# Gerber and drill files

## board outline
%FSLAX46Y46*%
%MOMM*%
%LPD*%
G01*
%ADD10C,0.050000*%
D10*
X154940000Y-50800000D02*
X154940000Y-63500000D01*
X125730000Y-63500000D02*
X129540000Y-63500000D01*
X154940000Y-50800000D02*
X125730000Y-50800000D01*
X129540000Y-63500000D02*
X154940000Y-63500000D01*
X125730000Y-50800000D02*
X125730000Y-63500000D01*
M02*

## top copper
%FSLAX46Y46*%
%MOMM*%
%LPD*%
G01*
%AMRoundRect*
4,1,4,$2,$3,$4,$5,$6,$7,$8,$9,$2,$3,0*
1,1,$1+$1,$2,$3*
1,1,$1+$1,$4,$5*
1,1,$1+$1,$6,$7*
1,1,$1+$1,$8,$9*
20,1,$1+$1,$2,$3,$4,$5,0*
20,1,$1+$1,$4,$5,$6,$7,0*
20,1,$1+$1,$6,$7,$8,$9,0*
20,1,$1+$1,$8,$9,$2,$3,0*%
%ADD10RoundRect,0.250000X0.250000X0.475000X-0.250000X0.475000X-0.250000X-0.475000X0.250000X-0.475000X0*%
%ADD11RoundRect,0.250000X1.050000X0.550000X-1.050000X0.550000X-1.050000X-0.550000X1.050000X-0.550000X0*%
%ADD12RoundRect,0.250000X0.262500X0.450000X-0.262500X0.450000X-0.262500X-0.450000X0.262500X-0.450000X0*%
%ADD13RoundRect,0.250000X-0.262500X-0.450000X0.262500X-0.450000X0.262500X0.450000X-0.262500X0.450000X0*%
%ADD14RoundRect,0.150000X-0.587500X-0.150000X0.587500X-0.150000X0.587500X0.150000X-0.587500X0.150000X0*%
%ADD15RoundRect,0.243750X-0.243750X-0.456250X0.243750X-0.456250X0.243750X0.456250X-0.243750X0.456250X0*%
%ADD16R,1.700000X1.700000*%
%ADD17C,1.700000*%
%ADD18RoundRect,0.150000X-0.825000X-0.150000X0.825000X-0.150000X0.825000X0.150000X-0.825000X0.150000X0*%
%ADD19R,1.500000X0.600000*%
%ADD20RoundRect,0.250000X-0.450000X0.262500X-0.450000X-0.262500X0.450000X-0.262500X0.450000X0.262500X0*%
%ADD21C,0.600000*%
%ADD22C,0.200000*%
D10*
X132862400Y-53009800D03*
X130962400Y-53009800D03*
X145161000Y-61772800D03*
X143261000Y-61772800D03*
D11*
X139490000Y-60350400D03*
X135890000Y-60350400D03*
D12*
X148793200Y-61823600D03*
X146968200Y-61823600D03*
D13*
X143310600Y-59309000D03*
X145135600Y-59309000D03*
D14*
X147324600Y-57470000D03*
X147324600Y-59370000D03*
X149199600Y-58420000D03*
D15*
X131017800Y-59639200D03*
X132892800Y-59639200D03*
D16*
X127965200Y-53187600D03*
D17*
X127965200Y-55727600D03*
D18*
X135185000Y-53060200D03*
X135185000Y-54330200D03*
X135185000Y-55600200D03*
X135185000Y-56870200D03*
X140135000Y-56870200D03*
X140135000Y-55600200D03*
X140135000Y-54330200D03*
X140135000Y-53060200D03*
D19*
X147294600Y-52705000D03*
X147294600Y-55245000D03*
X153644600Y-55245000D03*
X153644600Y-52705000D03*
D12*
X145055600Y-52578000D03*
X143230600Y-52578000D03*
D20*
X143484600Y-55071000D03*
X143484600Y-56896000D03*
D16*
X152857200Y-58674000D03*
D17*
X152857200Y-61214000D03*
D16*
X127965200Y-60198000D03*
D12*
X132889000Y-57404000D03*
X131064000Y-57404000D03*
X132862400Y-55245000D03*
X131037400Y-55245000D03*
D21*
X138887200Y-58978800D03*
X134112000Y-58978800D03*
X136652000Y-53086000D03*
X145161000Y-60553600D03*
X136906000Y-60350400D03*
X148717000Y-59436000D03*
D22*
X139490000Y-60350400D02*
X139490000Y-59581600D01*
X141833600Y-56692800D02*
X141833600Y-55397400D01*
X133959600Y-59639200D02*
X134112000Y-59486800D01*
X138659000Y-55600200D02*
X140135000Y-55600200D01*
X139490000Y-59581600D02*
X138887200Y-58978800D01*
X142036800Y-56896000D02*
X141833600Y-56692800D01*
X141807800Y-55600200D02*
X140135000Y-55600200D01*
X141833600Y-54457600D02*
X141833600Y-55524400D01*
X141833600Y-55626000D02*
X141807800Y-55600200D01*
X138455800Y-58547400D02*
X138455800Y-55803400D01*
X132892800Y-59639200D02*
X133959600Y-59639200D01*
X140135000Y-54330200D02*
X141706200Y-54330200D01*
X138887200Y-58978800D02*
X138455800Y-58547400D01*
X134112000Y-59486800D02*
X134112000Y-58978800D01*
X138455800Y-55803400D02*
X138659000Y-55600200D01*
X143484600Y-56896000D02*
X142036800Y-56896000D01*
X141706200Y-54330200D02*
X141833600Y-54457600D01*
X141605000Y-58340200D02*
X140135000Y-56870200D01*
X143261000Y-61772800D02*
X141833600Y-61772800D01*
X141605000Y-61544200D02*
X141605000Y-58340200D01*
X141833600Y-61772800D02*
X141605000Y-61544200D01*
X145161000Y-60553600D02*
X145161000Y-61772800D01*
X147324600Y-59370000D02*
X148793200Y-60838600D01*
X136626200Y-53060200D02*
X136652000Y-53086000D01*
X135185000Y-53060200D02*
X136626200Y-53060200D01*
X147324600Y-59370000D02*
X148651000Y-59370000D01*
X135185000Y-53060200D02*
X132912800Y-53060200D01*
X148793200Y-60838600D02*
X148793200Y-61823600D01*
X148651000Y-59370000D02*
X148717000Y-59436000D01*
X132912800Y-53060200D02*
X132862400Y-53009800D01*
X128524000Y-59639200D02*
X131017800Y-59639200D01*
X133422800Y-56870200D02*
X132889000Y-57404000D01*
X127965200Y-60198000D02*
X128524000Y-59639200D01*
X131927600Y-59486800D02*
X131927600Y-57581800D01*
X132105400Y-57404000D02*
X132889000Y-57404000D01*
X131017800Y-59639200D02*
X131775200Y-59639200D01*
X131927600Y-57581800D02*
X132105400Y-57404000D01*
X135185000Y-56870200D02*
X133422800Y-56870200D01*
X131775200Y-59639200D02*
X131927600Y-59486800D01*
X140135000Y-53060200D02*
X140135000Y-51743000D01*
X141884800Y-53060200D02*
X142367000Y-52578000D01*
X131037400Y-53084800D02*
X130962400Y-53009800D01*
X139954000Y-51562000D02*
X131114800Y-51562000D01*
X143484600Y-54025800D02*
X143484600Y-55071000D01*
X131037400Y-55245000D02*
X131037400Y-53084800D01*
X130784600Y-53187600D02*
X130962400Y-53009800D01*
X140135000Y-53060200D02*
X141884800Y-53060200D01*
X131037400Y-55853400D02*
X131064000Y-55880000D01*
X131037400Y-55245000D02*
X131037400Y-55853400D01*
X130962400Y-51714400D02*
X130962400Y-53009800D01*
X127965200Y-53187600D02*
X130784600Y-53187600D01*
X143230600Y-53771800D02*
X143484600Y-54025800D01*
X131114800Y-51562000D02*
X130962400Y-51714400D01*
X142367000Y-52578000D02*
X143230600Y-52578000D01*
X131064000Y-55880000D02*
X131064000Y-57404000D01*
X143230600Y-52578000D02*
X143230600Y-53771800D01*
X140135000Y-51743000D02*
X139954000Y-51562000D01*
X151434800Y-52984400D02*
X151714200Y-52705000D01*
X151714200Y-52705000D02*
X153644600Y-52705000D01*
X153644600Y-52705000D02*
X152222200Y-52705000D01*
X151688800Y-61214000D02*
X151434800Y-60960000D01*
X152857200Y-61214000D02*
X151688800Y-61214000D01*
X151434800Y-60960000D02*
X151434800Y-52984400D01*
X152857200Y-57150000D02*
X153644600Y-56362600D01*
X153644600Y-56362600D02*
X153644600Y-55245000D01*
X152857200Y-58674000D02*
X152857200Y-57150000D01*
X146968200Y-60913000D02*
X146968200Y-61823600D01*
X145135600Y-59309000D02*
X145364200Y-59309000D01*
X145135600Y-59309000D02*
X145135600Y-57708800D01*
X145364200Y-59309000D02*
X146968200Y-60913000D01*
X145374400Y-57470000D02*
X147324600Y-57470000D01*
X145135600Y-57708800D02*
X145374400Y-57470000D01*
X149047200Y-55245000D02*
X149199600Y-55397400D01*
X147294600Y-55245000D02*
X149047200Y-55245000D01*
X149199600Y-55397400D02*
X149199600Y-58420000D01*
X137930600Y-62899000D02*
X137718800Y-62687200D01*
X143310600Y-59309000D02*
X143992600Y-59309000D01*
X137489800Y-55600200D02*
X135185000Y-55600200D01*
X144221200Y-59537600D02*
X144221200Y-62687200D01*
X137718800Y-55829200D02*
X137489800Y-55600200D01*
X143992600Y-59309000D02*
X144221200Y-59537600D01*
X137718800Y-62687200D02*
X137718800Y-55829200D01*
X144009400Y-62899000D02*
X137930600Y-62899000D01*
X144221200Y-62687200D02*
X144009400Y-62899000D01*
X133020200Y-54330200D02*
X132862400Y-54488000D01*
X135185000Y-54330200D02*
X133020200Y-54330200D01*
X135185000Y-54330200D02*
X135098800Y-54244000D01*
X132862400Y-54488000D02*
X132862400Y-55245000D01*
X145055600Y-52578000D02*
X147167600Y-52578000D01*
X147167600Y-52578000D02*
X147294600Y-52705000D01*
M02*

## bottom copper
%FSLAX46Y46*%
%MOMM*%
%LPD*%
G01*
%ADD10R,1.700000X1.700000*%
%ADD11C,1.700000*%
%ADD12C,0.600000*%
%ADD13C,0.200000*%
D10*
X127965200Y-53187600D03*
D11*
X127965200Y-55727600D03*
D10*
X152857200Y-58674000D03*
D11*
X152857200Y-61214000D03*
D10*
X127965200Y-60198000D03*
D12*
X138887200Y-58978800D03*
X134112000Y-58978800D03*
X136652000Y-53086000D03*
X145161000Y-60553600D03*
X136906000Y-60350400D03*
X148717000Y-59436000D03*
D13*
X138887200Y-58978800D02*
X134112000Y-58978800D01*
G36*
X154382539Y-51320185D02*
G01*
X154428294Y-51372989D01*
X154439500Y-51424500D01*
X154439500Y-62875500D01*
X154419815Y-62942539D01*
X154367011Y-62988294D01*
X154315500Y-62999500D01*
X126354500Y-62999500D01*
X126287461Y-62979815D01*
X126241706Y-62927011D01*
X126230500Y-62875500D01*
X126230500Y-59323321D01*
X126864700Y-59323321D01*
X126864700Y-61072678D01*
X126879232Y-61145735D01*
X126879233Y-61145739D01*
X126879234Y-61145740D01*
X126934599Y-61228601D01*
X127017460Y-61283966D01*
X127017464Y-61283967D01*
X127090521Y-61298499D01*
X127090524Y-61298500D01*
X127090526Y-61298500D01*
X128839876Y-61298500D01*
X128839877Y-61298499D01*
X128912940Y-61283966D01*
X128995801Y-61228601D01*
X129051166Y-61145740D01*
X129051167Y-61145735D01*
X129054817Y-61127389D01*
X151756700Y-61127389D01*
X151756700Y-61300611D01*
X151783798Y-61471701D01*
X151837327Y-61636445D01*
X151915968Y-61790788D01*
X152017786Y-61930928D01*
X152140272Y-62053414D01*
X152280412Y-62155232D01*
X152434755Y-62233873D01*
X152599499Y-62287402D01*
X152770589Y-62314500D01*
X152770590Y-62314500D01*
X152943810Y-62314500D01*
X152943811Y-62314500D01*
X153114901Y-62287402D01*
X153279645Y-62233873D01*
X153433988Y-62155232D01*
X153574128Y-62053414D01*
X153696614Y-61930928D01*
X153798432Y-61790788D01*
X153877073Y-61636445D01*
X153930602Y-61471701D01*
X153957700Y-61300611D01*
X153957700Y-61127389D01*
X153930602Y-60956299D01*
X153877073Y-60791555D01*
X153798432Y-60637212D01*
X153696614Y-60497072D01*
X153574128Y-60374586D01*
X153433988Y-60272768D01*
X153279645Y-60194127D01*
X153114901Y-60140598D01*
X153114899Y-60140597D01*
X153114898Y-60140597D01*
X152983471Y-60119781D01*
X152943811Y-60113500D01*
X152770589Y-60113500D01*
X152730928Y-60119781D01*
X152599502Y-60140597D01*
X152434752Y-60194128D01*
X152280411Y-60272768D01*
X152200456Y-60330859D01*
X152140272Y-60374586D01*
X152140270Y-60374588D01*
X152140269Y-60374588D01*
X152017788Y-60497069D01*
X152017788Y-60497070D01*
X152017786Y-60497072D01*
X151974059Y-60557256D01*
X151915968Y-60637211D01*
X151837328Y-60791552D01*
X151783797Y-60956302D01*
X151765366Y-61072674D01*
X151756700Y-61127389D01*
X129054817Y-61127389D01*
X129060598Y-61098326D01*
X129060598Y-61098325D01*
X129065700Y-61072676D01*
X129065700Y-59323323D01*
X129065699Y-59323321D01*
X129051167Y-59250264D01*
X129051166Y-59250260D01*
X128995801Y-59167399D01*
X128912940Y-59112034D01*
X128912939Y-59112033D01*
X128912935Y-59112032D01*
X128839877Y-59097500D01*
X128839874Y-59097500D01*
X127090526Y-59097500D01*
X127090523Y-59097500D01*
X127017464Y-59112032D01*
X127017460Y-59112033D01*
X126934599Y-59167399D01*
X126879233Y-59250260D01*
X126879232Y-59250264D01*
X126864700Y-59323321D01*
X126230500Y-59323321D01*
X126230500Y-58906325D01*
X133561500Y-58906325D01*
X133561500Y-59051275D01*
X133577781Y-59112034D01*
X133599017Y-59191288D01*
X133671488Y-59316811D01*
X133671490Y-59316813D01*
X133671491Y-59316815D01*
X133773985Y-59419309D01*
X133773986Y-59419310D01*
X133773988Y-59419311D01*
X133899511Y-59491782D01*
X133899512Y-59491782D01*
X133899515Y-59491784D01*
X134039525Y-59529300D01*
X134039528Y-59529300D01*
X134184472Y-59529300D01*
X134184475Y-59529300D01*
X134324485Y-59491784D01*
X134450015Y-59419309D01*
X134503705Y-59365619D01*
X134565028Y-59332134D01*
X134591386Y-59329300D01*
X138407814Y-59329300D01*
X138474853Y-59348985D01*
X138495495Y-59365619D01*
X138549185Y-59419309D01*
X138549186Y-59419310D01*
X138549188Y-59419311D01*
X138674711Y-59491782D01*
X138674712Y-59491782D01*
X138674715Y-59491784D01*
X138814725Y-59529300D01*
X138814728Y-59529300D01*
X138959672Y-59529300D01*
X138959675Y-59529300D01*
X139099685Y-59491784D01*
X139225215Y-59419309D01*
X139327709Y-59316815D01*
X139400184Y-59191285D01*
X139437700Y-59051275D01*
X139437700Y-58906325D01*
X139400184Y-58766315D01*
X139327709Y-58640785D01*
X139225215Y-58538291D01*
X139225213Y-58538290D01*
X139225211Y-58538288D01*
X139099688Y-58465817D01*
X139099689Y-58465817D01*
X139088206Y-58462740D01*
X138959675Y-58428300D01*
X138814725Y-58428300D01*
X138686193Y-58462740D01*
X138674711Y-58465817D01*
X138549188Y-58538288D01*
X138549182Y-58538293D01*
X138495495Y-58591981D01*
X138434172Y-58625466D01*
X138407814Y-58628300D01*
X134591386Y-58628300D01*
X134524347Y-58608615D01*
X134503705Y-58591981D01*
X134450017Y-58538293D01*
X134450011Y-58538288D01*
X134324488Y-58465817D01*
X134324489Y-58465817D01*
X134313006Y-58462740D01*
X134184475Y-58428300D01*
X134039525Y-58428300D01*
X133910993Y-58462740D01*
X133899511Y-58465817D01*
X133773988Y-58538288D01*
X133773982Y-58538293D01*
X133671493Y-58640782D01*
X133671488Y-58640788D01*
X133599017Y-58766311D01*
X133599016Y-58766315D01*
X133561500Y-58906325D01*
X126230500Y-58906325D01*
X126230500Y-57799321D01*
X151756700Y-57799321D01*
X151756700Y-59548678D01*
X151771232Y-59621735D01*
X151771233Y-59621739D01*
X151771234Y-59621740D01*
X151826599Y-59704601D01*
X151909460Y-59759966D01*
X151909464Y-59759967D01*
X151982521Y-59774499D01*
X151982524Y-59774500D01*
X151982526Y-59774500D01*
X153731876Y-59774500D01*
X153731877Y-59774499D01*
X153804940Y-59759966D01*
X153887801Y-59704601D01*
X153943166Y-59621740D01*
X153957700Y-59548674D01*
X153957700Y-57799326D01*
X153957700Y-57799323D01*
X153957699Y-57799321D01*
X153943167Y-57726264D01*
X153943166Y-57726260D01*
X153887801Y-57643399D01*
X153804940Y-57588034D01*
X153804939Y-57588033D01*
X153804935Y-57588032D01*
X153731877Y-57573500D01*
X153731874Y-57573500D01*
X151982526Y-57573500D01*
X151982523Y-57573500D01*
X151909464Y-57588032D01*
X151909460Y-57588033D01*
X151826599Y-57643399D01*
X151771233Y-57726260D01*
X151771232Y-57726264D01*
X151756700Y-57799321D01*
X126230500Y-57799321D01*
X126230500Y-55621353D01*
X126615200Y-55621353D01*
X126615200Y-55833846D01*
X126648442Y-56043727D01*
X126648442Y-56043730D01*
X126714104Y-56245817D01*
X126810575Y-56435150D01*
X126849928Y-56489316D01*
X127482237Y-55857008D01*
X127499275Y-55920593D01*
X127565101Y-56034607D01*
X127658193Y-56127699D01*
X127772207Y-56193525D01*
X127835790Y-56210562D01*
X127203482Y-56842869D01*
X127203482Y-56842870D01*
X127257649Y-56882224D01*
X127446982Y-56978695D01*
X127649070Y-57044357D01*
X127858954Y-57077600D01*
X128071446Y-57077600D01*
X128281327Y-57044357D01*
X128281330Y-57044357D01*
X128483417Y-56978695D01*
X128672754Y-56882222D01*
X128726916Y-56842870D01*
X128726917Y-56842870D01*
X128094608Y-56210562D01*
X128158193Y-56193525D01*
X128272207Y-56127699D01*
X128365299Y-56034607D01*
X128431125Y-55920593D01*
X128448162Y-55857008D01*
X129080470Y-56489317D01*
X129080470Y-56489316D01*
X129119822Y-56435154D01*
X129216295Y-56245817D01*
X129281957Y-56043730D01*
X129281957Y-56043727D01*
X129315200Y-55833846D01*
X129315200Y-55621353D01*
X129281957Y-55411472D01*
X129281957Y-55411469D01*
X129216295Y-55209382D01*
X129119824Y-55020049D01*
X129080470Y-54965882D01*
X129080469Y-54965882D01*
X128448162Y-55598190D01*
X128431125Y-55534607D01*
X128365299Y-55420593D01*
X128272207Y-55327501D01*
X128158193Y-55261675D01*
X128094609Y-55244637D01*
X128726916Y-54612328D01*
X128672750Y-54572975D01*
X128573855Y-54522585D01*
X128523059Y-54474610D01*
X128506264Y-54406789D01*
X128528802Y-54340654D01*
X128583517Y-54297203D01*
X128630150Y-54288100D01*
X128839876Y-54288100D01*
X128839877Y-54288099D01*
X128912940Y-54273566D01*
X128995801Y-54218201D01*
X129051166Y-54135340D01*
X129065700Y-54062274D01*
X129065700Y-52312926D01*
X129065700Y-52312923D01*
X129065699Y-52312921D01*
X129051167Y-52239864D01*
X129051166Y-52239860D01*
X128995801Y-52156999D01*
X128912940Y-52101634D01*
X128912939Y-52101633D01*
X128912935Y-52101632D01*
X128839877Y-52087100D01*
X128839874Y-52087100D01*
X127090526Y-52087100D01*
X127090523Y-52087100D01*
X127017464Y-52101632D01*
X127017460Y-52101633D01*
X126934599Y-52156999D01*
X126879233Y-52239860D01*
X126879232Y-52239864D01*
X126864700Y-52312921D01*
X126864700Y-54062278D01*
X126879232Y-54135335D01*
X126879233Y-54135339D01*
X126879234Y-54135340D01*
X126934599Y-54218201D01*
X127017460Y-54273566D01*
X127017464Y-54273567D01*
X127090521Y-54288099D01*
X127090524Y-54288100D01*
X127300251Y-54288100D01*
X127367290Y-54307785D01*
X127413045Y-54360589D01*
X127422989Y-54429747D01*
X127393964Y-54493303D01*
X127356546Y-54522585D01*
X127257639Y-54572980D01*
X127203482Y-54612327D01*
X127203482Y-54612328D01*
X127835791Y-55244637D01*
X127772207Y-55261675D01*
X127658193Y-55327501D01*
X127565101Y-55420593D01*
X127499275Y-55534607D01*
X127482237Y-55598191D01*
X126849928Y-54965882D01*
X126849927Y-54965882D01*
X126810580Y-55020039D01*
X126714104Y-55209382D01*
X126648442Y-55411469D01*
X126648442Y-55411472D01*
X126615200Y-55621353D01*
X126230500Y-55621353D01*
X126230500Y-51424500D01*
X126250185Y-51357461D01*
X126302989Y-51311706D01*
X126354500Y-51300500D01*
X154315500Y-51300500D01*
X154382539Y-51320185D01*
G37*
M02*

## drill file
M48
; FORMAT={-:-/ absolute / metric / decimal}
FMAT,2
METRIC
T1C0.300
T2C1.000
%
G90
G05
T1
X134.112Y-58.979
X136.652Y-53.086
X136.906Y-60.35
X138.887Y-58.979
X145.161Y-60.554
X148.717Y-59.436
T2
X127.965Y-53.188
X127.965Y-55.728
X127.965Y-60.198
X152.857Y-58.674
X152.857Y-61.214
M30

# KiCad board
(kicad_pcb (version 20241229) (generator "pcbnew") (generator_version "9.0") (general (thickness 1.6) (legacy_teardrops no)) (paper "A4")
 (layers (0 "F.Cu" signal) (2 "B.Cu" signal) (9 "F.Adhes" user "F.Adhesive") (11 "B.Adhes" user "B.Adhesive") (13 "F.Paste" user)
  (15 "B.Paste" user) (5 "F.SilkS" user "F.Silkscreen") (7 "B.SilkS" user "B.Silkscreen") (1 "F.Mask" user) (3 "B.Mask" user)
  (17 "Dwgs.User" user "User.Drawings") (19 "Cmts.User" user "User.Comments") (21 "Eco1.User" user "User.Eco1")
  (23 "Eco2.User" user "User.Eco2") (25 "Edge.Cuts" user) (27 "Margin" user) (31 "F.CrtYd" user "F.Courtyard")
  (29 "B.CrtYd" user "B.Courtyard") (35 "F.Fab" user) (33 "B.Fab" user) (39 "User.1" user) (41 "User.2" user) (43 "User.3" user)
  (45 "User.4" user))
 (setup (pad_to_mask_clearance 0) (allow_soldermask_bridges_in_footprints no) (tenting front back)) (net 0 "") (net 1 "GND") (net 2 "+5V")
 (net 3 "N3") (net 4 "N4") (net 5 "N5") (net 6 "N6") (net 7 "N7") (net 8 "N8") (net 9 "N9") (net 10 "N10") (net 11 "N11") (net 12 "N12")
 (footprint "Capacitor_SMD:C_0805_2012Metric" (layer "F.Cu") (at 131.9124 53.0098 180)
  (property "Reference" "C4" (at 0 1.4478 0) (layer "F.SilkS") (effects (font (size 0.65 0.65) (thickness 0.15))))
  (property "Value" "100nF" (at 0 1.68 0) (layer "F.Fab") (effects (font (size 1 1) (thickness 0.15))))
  (pad "1" smd roundrect (at -0.95 0 180) (size 1 1.45) (layers "F.Cu" "F.Mask" "F.Paste") (roundrect_rratio 0.25) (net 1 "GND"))
  (pad "2" smd roundrect (at 0.95 0 180) (size 1 1.45) (layers "F.Cu" "F.Mask" "F.Paste") (roundrect_rratio 0.25) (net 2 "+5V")))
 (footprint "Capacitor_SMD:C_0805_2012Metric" (layer "F.Cu") (at 144.211 61.7728 180)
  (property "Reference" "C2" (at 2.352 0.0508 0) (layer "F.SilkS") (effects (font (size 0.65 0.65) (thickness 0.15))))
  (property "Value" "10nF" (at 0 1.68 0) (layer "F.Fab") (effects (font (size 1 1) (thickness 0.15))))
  (pad "1" smd roundrect (at -0.95 0 180) (size 1 1.45) (layers "F.Cu" "F.Mask" "F.Paste") (roundrect_rratio 0.25) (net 1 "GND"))
  (pad "2" smd roundrect (at 0.95 0 180) (size 1 1.45) (layers "F.Cu" "F.Mask" "F.Paste") (roundrect_rratio 0.25) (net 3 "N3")))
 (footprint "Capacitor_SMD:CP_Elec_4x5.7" (layer "F.Cu") (at 137.69 60.3504 180)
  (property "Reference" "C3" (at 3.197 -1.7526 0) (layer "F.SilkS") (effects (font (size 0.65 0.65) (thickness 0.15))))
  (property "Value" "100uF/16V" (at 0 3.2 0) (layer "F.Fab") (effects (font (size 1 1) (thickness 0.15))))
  (pad "1" smd roundrect (at -1.8 0 180) (size 2.6 1.6) (layers "F.Cu" "F.Mask" "F.Paste") (roundrect_rratio 0.15625) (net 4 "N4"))
  (pad "2" smd roundrect (at 1.8 0 180) (size 2.6 1.6) (layers "F.Cu" "F.Mask" "F.Paste") (roundrect_rratio 0.15625) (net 1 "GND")))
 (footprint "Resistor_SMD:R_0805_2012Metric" (layer "F.Cu") (at 147.8807 61.8236 180)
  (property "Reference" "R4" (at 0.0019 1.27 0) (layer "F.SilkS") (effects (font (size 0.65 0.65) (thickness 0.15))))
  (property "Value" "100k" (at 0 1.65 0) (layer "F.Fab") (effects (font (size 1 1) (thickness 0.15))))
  (pad "1" smd roundrect (at -0.9125 0 180) (size 1.025 1.4) (layers "F.Cu" "F.Mask" "F.Paste") (roundrect_rratio 0.243902) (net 1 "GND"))
  (pad "2" smd roundrect (at 0.9125 0 180) (size 1.025 1.4) (layers "F.Cu" "F.Mask" "F.Paste") (roundrect_rratio 0.243902) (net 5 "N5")))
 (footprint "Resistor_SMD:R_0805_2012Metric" (layer "F.Cu") (at 144.2231 59.309)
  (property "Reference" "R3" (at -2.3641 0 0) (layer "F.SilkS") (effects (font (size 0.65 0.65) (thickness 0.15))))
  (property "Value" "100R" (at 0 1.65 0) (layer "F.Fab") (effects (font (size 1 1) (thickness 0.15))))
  (pad "1" smd roundrect (at -0.9125 0) (size 1.025 1.4) (layers "F.Cu" "F.Mask" "F.Paste") (roundrect_rratio 0.243902) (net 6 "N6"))
  (pad "2" smd roundrect (at 0.9125 0) (size 1.025 1.4) (layers "F.Cu" "F.Mask" "F.Paste") (roundrect_rratio 0.243902) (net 5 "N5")))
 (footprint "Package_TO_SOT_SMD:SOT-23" (layer "F.Cu") (at 148.2621 58.42)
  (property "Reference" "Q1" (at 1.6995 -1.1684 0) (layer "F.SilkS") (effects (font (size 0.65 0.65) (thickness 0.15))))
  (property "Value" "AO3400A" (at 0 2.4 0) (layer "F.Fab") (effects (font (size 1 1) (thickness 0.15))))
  (pad "1" smd roundrect (at -0.9375 -0.95) (size 1.475 0.6) (layers "F.Cu" "F.Mask" "F.Paste") (roundrect_rratio 0.25) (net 5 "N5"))
  (pad "2" smd roundrect (at -0.9375 0.95) (size 1.475 0.6) (layers "F.Cu" "F.Mask" "F.Paste") (roundrect_rratio 0.25) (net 1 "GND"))
  (pad "3" smd roundrect (at 0.9375 0) (size 1.475 0.6) (layers "F.Cu" "F.Mask" "F.Paste") (roundrect_rratio 0.25) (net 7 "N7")))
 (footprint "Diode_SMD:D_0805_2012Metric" (layer "F.Cu") (at 131.9553 59.6392)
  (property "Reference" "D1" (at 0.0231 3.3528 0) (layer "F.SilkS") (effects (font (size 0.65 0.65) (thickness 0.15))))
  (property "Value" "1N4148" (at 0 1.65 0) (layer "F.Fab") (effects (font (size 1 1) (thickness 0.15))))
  (pad "1" smd roundrect (at -0.9375 0) (size 0.975 1.4) (layers "F.Cu" "F.Mask" "F.Paste") (roundrect_rratio 0.25) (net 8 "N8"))
  (pad "2" smd roundrect (at 0.9375 0) (size 0.975 1.4) (layers "F.Cu" "F.Mask" "F.Paste") (roundrect_rratio 0.25) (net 4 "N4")))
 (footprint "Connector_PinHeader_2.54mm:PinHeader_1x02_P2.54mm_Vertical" (layer "F.Cu") (at 127.9652 53.1876)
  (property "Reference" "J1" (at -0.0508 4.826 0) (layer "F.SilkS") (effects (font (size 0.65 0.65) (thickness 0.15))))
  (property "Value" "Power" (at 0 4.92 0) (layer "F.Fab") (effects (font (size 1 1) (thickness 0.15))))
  (pad "1" thru_hole rect (at 0 0) (size 1.7 1.7) (drill 1) (layers "*.Cu" "*.Mask") (remove_unused_layers no) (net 2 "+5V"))
  (pad "2" thru_hole circle (at 0 2.54) (size 1.7 1.7) (drill 1) (layers "*.Cu" "*.Mask") (remove_unused_layers no) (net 1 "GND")))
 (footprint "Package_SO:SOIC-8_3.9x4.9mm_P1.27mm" (layer "F.Cu") (at 137.66 54.9652)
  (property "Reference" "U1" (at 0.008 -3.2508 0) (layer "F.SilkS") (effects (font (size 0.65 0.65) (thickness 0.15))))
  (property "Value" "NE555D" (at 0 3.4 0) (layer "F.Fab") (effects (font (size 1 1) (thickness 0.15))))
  (pad "1" smd roundrect (at -2.475 -1.905) (size 1.95 0.6) (layers "F.Cu" "F.Mask" "F.Paste") (roundrect_rratio 0.25) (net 1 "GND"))
  (pad "2" smd roundrect (at -2.475 -0.635) (size 1.95 0.6) (layers "F.Cu" "F.Mask" "F.Paste") (roundrect_rratio 0.25) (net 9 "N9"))
  (pad "3" smd roundrect (at -2.475 0.635) (size 1.95 0.6) (layers "F.Cu" "F.Mask" "F.Paste") (roundrect_rratio 0.25) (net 6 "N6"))
  (pad "4" smd roundrect (at -2.475 1.905) (size 1.95 0.6) (layers "F.Cu" "F.Mask" "F.Paste") (roundrect_rratio 0.25) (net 8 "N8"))
  (pad "5" smd roundrect (at 2.475 1.905) (size 1.95 0.6) (layers "F.Cu" "F.Mask" "F.Paste") (roundrect_rratio 0.25) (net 3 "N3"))
  (pad "6" smd roundrect (at 2.475 0.635) (size 1.95 0.6) (layers "F.Cu" "F.Mask" "F.Paste") (roundrect_rratio 0.25) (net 4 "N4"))
  (pad "7" smd roundrect (at 2.475 -0.635) (size 1.95 0.6) (layers "F.Cu" "F.Mask" "F.Paste") (roundrect_rratio 0.25) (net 4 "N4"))
  (pad "8" smd roundrect (at 2.475 -1.905) (size 1.95 0.6) (layers "F.Cu" "F.Mask" "F.Paste") (roundrect_rratio 0.25) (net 2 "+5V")))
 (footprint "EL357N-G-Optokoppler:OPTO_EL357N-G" (layer "F.Cu") (at 150.4696 53.975)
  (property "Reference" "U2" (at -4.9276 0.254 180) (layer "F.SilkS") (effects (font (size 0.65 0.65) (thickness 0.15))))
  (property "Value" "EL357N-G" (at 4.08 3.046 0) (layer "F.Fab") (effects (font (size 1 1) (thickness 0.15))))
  (pad "1" smd rect (at -3.175 -1.27) (size 1.5 0.6) (layers "F.Cu" "F.Mask" "F.Paste") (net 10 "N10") (solder_mask_margin 0.102))
  (pad "2" smd rect (at -3.175 1.27) (size 1.5 0.6) (layers "F.Cu" "F.Mask" "F.Paste") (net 7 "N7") (solder_mask_margin 0.102))
  (pad "3" smd rect (at 3.175 1.27) (size 1.5 0.6) (layers "F.Cu" "F.Mask" "F.Paste") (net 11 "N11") (solder_mask_margin 0.102))
  (pad "4" smd rect (at 3.175 -1.27) (size 1.5 0.6) (layers "F.Cu" "F.Mask" "F.Paste") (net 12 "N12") (solder_mask_margin 0.102)))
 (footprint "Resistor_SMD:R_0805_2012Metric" (layer "F.Cu") (at 144.1431 52.578 180)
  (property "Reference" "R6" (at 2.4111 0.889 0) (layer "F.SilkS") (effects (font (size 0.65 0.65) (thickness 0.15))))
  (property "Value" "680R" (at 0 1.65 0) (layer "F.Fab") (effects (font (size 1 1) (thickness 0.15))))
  (pad "1" smd roundrect (at -0.9125 0 180) (size 1.025 1.4) (layers "F.Cu" "F.Mask" "F.Paste") (roundrect_rratio 0.243902) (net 10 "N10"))
  (pad "2" smd roundrect (at 0.9125 0 180) (size 1.025 1.4) (layers "F.Cu" "F.Mask" "F.Paste") (roundrect_rratio 0.243902) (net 2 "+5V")))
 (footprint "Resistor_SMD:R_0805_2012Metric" (layer "F.Cu") (at 143.4846 55.9835 -90)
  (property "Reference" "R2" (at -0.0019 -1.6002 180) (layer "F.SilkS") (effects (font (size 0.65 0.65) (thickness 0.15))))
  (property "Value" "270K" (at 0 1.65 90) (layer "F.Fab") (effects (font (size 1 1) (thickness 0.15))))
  (pad "1" smd roundrect (at -0.9125 0 270) (size 1.025 1.4) (layers "F.Cu" "F.Mask" "F.Paste") (roundrect_rratio 0.243902) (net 2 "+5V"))
  (pad "2" smd roundrect (at 0.9125 0 270) (size 1.025 1.4) (layers "F.Cu" "F.Mask" "F.Paste") (roundrect_rratio 0.243902) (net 4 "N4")))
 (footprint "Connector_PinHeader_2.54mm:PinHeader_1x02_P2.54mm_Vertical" (layer "F.Cu") (at 152.8572 58.674)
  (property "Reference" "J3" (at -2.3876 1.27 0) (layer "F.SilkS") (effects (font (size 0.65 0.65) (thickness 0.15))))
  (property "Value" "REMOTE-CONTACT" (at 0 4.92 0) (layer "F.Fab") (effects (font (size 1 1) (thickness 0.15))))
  (pad "1" thru_hole rect (at 0 0) (size 1.7 1.7) (drill 1) (layers "*.Cu" "*.Mask") (remove_unused_layers no) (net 11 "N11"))
  (pad "2" thru_hole circle (at 0 2.54) (size 1.7 1.7) (drill 1) (layers "*.Cu" "*.Mask") (remove_unused_layers no) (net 12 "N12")))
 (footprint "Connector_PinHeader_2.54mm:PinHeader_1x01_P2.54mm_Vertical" (layer "F.Cu") (at 127.9652 60.198 180)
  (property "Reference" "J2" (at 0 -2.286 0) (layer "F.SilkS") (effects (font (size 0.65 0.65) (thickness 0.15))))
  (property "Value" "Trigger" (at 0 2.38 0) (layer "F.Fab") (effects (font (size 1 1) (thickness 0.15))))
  (pad "1" thru_hole rect (at 0 0 180) (size 1.7 1.7) (drill 1) (layers "*.Cu" "*.Mask") (remove_unused_layers no) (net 8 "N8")))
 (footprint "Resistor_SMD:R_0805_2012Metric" (layer "F.Cu") (at 131.9765 57.404 180)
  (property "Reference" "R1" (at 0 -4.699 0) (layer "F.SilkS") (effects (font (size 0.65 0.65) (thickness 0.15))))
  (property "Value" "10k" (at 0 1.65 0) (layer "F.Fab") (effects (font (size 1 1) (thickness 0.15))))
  (pad "1" smd roundrect (at -0.9125 0 180) (size 1.025 1.4) (layers "F.Cu" "F.Mask" "F.Paste") (roundrect_rratio 0.243902) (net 8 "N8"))
  (pad "2" smd roundrect (at 0.9125 0 180) (size 1.025 1.4) (layers "F.Cu" "F.Mask" "F.Paste") (roundrect_rratio 0.243902) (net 2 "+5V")))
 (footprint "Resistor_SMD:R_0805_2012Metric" (layer "F.Cu") (at 131.9499 55.245 180)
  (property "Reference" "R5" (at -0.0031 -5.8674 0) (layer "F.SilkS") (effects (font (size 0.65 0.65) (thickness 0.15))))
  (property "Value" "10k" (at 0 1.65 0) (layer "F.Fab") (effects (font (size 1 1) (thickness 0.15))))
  (pad "1" smd roundrect (at -0.9125 0 180) (size 1.025 1.4) (layers "F.Cu" "F.Mask" "F.Paste") (roundrect_rratio 0.243902) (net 9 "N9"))
  (pad "2" smd roundrect (at 0.9125 0 180) (size 1.025 1.4) (layers "F.Cu" "F.Mask" "F.Paste") (roundrect_rratio 0.243902) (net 2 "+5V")))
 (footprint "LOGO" (layer "B.Cu") (at 140.97 57.5056 180)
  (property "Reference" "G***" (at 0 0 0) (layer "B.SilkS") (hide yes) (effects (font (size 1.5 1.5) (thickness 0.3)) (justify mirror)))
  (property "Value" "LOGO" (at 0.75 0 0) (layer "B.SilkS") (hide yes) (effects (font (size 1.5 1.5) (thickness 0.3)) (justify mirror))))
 (gr_line (start 154.94 50.8) (end 154.94 63.5) (stroke (width 0.05) (type default)) (layer "Edge.Cuts"))
 (gr_line (start 125.73 63.5) (end 129.54 63.5) (stroke (width 0.05) (type default)) (layer "Edge.Cuts"))
 (gr_line (start 154.94 50.8) (end 125.73 50.8) (stroke (width 0.05) (type default)) (layer "Edge.Cuts"))
 (gr_line (start 129.54 63.5) (end 154.94 63.5) (stroke (width 0.05) (type default)) (layer "Edge.Cuts"))
 (gr_line (start 125.73 50.8) (end 125.73 63.5) (stroke (width 0.05) (type default)) (layer "Edge.Cuts"))
 (segment (start 139.49 60.3504) (end 139.49 59.5816) (width 0.2) (layer "F.Cu") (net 4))
 (segment (start 141.8336 56.6928) (end 141.8336 55.3974) (width 0.2) (layer "F.Cu") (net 4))
 (segment (start 133.9596 59.6392) (end 134.112 59.4868) (width 0.2) (layer "F.Cu") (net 4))
 (segment (start 138.659 55.6002) (end 140.135 55.6002) (width 0.2) (layer "F.Cu") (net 4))
 (segment (start 139.49 59.5816) (end 138.8872 58.9788) (width 0.2) (layer "F.Cu") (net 4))
 (segment (start 142.0368 56.896) (end 141.8336 56.6928) (width 0.2) (layer "F.Cu") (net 4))
 (segment (start 141.8078 55.6002) (end 140.135 55.6002) (width 0.2) (layer "F.Cu") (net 4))
 (segment (start 141.8336 54.4576) (end 141.8336 55.5244) (width 0.2) (layer "F.Cu") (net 4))
 (segment (start 141.8336 55.626) (end 141.8078 55.6002) (width 0.2) (layer "F.Cu") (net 4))
 (segment (start 138.4558 58.5474) (end 138.4558 55.8034) (width 0.2) (layer "F.Cu") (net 4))
 (segment (start 132.8928 59.6392) (end 133.9596 59.6392) (width 0.2) (layer "F.Cu") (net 4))
 (segment (start 140.135 54.3302) (end 141.7062 54.3302) (width 0.2) (layer "F.Cu") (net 4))
 (segment (start 138.8872 58.9788) (end 138.4558 58.5474) (width 0.2) (layer "F.Cu") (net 4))
 (segment (start 134.112 59.4868) (end 134.112 58.9788) (width 0.2) (layer "F.Cu") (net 4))
 (segment (start 138.4558 55.8034) (end 138.659 55.6002) (width 0.2) (layer "F.Cu") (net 4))
 (segment (start 143.4846 56.896) (end 142.0368 56.896) (width 0.2) (layer "F.Cu") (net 4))
 (segment (start 141.7062 54.3302) (end 141.8336 54.4576) (width 0.2) (layer "F.Cu") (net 4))
 (via (at 138.8872 58.9788) (size 0.6) (drill 0.3) (layers "F.Cu" "B.Cu") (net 4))
 (via (at 134.112 58.9788) (size 0.6) (drill 0.3) (layers "F.Cu" "B.Cu") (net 4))
 (segment (start 138.8872 58.9788) (end 134.112 58.9788) (width 0.2) (layer "B.Cu") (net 4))
 (segment (start 141.605 58.3402) (end 140.135 56.8702) (width 0.2) (layer "F.Cu") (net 3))
 (segment (start 143.261 61.7728) (end 141.8336 61.7728) (width 0.2) (layer "F.Cu") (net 3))
 (segment (start 141.605 61.5442) (end 141.605 58.3402) (width 0.2) (layer "F.Cu") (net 3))
 (segment (start 141.8336 61.7728) (end 141.605 61.5442) (width 0.2) (layer "F.Cu") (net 3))
 (segment (start 145.161 60.5536) (end 145.161 61.7728) (width 0.2) (layer "F.Cu") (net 1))
 (segment (start 147.3246 59.37) (end 148.7932 60.8386) (width 0.2) (layer "F.Cu") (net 1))
 (segment (start 136.6262 53.0602) (end 136.652 53.086) (width 0.2) (layer "F.Cu") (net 1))
 (segment (start 135.185 53.0602) (end 136.6262 53.0602) (width 0.2) (layer "F.Cu") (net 1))
 (segment (start 147.3246 59.37) (end 148.651 59.37) (width 0.2) (layer "F.Cu") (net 1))
 (segment (start 135.185 53.0602) (end 132.9128 53.0602) (width 0.2) (layer "F.Cu") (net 1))
 (segment (start 148.7932 60.8386) (end 148.7932 61.8236) (width 0.2) (layer "F.Cu") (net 1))
 (segment (start 148.651 59.37) (end 148.717 59.436) (width 0.2) (layer "F.Cu") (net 1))
 (segment (start 132.9128 53.0602) (end 132.8624 53.0098) (width 0.2) (layer "F.Cu") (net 1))
 (via (at 136.652 53.086) (size 0.6) (drill 0.3) (layers "F.Cu" "B.Cu") (free yes) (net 1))
 (via (at 145.161 60.5536) (size 0.6) (drill 0.3) (layers "F.Cu" "B.Cu") (free yes) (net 1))
 (via (at 136.906 60.3504) (size 0.6) (drill 0.3) (layers "F.Cu" "B.Cu") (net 1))
 (via (at 148.717 59.436) (size 0.6) (drill 0.3) (layers "F.Cu" "B.Cu") (free yes) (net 1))
 (segment (start 128.524 59.6392) (end 131.0178 59.6392) (width 0.2) (layer "F.Cu") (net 8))
 (segment (start 133.4228 56.8702) (end 132.889 57.404) (width 0.2) (layer "F.Cu") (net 8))
 (segment (start 127.9652 60.198) (end 128.524 59.6392) (width 0.2) (layer "F.Cu") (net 8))
 (segment (start 131.9276 59.4868) (end 131.9276 57.5818) (width 0.2) (layer "F.Cu") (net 8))
 (segment (start 132.1054 57.404) (end 132.889 57.404) (width 0.2) (layer "F.Cu") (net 8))
 (segment (start 131.0178 59.6392) (end 131.7752 59.6392) (width 0.2) (layer "F.Cu") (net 8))
 (segment (start 131.9276 57.5818) (end 132.1054 57.404) (width 0.2) (layer "F.Cu") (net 8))
 (segment (start 135.185 56.8702) (end 133.4228 56.8702) (width 0.2) (layer "F.Cu") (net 8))
 (segment (start 131.7752 59.6392) (end 131.9276 59.4868) (width 0.2) (layer "F.Cu") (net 8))
 (segment (start 140.135 53.0602) (end 140.135 51.743) (width 0.2) (layer "F.Cu") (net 2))
 (segment (start 141.8848 53.0602) (end 142.367 52.578) (width 0.2) (layer "F.Cu") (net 2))
 (segment (start 131.0374 53.0848) (end 130.9624 53.0098) (width 0.2) (layer "F.Cu") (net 2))
 (segment (start 139.954 51.562) (end 131.1148 51.562) (width 0.2) (layer "F.Cu") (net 2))
 (segment (start 143.4846 54.0258) (end 143.4846 55.071) (width 0.2) (layer "F.Cu") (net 2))
 (segment (start 131.0374 55.245) (end 131.0374 53.0848) (width 0.2) (layer "F.Cu") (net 2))
 (segment (start 130.7846 53.1876) (end 130.9624 53.0098) (width 0.2) (layer "F.Cu") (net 2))
 (segment (start 140.135 53.0602) (end 141.8848 53.0602) (width 0.2) (layer "F.Cu") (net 2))
 (segment (start 131.0374 55.8534) (end 131.064 55.88) (width 0.2) (layer "F.Cu") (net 2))
 (segment (start 131.0374 55.245) (end 131.0374 55.8534) (width 0.2) (layer "F.Cu") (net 2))
 (segment (start 130.9624 51.7144) (end 130.9624 53.0098) (width 0.2) (layer "F.Cu") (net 2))
 (segment (start 127.9652 53.1876) (end 130.7846 53.1876) (width 0.2) (layer "F.Cu") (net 2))
 (segment (start 143.2306 53.7718) (end 143.4846 54.0258) (width 0.2) (layer "F.Cu") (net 2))
 (segment (start 131.1148 51.562) (end 130.9624 51.7144) (width 0.2) (layer "F.Cu") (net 2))
 (segment (start 142.367 52.578) (end 143.2306 52.578) (width 0.2) (layer "F.Cu") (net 2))
 (segment (start 131.064 55.88) (end 131.064 57.404) (width 0.2) (layer "F.Cu") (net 2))
 (segment (start 143.2306 52.578) (end 143.2306 53.7718) (width 0.2) (layer "F.Cu") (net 2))
 (segment (start 140.135 51.743) (end 139.954 51.562) (width 0.2) (layer "F.Cu") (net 2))
 (segment (start 151.4348 52.9844) (end 151.7142 52.705) (width 0.2) (layer "F.Cu") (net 12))
 (segment (start 151.7142 52.705) (end 153.6446 52.705) (width 0.2) (layer "F.Cu") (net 12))
 (segment (start 153.6446 52.705) (end 152.2222 52.705) (width 0.2) (layer "F.Cu") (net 12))
 (segment (start 151.6888 61.214) (end 151.4348 60.96) (width 0.2) (layer "F.Cu") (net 12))
 (segment (start 152.8572 61.214) (end 151.6888 61.214) (width 0.2) (layer "F.Cu") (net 12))
 (segment (start 151.4348 60.96) (end 151.4348 52.9844) (width 0.2) (layer "F.Cu") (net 12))
 (segment (start 152.8572 57.15) (end 153.6446 56.3626) (width 0.2) (layer "F.Cu") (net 11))
 (segment (start 153.6446 56.3626) (end 153.6446 55.245) (width 0.2) (layer "F.Cu") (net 11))
 (segment (start 152.8572 58.674) (end 152.8572 57.15) (width 0.2) (layer "F.Cu") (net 11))
 (segment (start 146.9682 60.913) (end 146.9682 61.8236) (width 0.2) (layer "F.Cu") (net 5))
 (segment (start 145.1356 59.309) (end 145.3642 59.309) (width 0.2) (layer "F.Cu") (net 5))
 (segment (start 145.1356 59.309) (end 145.1356 57.7088) (width 0.2) (layer "F.Cu") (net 5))
 (segment (start 145.3642 59.309) (end 146.9682 60.913) (width 0.2) (layer "F.Cu") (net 5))
 (segment (start 145.3744 57.47) (end 147.3246 57.47) (width 0.2) (layer "F.Cu") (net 5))
 (segment (start 145.1356 57.7088) (end 145.3744 57.47) (width 0.2) (layer "F.Cu") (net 5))
 (segment (start 149.0472 55.245) (end 149.1996 55.3974) (width 0.2) (layer "F.Cu") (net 7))
 (segment (start 147.2946 55.245) (end 149.0472 55.245) (width 0.2) (layer "F.Cu") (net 7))
 (segment (start 149.1996 55.3974) (end 149.1996 58.42) (width 0.2) (layer "F.Cu") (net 7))
 (segment (start 137.9306 62.899) (end 137.7188 62.6872) (width 0.2) (layer "F.Cu") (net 6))
 (segment (start 143.3106 59.309) (end 143.9926 59.309) (width 0.2) (layer "F.Cu") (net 6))
 (segment (start 137.4898 55.6002) (end 135.185 55.6002) (width 0.2) (layer "F.Cu") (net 6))
 (segment (start 144.2212 59.5376) (end 144.2212 62.6872) (width 0.2) (layer "F.Cu") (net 6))
 (segment (start 137.7188 55.8292) (end 137.4898 55.6002) (width 0.2) (layer "F.Cu") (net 6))
 (segment (start 143.9926 59.309) (end 144.2212 59.5376) (width 0.2) (layer "F.Cu") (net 6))
 (segment (start 137.7188 62.6872) (end 137.7188 55.8292) (width 0.2) (layer "F.Cu") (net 6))
 (segment (start 144.0094 62.899) (end 137.9306 62.899) (width 0.2) (layer "F.Cu") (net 6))
 (segment (start 144.2212 62.6872) (end 144.0094 62.899) (width 0.2) (layer "F.Cu") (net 6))
 (segment (start 133.0202 54.3302) (end 132.8624 54.488) (width 0.2) (layer "F.Cu") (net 9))
 (segment (start 135.185 54.3302) (end 133.0202 54.3302) (width 0.2) (layer "F.Cu") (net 9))
 (segment (start 135.185 54.3302) (end 135.0988 54.244) (width 0.2) (layer "F.Cu") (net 9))
 (segment (start 132.8624 54.488) (end 132.8624 55.245) (width 0.2) (layer "F.Cu") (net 9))
 (segment (start 145.0556 52.578) (end 147.1676 52.578) (width 0.2) (layer "F.Cu") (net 10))
 (segment (start 147.1676 52.578) (end 147.2946 52.705) (width 0.2) (layer "F.Cu") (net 10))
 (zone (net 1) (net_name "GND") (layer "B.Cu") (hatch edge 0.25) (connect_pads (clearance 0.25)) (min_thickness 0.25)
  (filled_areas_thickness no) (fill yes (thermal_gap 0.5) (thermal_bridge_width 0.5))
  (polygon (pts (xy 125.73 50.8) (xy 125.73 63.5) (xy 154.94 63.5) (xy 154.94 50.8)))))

